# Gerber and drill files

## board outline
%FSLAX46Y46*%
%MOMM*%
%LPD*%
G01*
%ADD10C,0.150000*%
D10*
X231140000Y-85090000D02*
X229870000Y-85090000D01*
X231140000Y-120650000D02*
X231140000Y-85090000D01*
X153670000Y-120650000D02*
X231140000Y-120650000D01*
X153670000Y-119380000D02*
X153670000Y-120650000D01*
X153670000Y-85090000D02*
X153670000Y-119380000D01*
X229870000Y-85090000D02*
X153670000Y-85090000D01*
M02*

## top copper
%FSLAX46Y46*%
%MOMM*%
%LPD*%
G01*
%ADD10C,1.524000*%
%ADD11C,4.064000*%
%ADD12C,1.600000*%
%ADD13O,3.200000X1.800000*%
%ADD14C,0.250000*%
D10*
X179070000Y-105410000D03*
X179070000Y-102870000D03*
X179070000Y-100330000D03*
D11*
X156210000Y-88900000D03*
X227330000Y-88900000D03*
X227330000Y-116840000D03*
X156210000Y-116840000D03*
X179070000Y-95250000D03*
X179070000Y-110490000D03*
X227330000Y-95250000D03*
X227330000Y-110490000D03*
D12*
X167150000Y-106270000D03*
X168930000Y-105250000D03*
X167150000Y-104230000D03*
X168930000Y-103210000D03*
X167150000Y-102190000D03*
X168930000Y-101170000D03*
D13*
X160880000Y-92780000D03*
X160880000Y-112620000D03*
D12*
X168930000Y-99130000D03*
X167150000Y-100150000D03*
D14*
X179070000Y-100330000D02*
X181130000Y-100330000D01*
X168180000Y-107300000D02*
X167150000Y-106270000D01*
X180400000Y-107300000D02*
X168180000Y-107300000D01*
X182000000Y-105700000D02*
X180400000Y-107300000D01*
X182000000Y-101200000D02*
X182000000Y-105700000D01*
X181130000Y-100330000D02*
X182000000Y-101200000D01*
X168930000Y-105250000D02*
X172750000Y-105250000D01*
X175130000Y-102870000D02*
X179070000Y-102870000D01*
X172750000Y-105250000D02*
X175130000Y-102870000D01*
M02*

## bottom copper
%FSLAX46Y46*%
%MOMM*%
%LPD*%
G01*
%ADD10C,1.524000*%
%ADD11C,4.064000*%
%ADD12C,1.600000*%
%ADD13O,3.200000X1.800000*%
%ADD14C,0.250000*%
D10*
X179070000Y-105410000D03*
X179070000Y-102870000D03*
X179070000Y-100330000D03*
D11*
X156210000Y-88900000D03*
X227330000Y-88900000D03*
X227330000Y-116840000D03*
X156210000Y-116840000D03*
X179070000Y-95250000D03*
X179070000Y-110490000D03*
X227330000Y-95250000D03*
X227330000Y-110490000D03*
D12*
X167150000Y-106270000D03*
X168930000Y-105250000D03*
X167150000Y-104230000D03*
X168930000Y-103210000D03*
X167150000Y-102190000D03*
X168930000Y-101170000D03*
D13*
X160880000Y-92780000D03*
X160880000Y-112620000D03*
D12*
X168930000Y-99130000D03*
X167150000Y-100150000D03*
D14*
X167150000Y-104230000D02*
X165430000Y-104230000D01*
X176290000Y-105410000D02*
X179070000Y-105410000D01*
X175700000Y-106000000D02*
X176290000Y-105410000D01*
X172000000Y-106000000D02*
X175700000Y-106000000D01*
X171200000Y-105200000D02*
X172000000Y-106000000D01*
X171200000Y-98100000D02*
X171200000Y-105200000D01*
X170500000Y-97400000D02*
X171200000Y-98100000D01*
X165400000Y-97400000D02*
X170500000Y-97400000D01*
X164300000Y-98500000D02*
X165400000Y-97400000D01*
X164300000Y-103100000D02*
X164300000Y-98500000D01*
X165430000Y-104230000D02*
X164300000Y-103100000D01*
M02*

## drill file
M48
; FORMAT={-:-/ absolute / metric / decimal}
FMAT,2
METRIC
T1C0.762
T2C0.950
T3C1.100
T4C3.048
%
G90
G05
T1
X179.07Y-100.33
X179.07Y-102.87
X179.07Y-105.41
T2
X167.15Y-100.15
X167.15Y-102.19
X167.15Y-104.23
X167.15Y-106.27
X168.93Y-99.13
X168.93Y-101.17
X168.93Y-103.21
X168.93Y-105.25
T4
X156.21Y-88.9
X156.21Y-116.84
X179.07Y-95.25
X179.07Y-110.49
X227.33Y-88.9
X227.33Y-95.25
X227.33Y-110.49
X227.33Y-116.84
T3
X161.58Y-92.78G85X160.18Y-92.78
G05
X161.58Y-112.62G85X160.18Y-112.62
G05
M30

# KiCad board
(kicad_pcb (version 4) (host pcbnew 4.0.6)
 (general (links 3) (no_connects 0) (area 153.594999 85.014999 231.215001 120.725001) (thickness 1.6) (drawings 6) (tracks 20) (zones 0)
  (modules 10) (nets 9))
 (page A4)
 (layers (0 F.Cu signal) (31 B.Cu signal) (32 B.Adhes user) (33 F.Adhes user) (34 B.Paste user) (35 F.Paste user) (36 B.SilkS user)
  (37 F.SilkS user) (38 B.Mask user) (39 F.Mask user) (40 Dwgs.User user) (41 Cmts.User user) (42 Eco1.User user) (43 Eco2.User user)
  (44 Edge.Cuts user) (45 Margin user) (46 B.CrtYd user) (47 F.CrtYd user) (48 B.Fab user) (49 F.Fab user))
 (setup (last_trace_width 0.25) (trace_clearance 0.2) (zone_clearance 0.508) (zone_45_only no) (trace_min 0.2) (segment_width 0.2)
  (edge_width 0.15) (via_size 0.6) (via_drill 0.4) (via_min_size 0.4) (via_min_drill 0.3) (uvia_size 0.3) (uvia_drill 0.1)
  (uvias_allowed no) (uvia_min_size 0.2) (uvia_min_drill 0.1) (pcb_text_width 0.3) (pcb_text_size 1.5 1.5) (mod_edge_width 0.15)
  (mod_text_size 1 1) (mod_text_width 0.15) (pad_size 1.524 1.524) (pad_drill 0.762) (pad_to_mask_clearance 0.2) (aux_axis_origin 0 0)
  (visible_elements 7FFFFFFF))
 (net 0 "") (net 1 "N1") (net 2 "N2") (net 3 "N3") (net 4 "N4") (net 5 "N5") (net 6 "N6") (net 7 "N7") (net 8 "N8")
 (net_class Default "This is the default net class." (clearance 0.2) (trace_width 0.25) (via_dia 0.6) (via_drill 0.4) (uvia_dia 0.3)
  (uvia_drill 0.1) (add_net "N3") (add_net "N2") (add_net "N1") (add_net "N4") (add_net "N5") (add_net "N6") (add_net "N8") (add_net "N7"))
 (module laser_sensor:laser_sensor (layer F.Cu) (at 176.53 102.87)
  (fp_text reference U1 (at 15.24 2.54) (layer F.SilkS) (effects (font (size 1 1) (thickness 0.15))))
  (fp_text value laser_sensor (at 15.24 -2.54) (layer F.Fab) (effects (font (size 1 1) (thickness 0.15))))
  (pad 1 thru_hole circle (at 2.54 2.54) (size 1.524 1.524) (drill 0.762) (layers *.Cu *.Mask) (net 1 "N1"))
  (pad 2 thru_hole circle (at 2.54 0) (size 1.524 1.524) (drill 0.762) (layers *.Cu *.Mask) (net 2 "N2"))
  (pad 3 thru_hole circle (at 2.54 -2.54) (size 1.524 1.524) (drill 0.762) (layers *.Cu *.Mask) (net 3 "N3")))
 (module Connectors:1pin (layer F.Cu) (at 156.21 88.9)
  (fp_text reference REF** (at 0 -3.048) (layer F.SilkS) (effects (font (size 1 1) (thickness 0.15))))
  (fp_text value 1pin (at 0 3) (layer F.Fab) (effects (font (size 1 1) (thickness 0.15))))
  (pad 1 thru_hole circle (at 0 0) (size 4.064 4.064) (drill 3.048) (layers *.Cu *.Mask)))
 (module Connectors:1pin (layer F.Cu) (at 227.33 88.9)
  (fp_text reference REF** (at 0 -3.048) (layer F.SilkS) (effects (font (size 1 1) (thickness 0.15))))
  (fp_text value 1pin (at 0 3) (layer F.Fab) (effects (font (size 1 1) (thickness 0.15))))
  (pad 1 thru_hole circle (at 0 0) (size 4.064 4.064) (drill 3.048) (layers *.Cu *.Mask)))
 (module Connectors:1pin (layer F.Cu) (at 227.33 116.84)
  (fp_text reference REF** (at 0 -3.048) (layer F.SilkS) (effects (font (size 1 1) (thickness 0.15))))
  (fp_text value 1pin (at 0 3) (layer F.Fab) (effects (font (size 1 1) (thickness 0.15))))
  (pad 1 thru_hole circle (at 0 0) (size 4.064 4.064) (drill 3.048) (layers *.Cu *.Mask)))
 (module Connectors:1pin (layer F.Cu) (at 156.21 116.84)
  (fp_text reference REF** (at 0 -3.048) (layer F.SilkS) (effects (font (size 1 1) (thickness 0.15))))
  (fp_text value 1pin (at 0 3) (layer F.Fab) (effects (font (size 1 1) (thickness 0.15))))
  (pad 1 thru_hole circle (at 0 0) (size 4.064 4.064) (drill 3.048) (layers *.Cu *.Mask)))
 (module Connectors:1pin (layer F.Cu) (at 179.07 95.25)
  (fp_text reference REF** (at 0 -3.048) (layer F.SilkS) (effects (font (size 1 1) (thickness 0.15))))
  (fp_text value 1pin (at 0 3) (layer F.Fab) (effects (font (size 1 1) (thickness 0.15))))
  (pad 1 thru_hole circle (at 0 0) (size 4.064 4.064) (drill 3.048) (layers *.Cu *.Mask)))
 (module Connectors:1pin (layer F.Cu) (at 179.07 110.49)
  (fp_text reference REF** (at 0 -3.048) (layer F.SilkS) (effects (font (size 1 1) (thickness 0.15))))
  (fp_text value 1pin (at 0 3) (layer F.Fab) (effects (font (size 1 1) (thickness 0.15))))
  (pad 1 thru_hole circle (at 0 0) (size 4.064 4.064) (drill 3.048) (layers *.Cu *.Mask)))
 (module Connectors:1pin (layer F.Cu) (at 227.33 95.25)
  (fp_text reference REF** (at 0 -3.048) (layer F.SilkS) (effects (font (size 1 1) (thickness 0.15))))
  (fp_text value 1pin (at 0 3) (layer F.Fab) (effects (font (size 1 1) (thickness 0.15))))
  (pad 1 thru_hole circle (at 0 0) (size 4.064 4.064) (drill 3.048) (layers *.Cu *.Mask)))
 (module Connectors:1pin (layer F.Cu) (at 227.33 110.49)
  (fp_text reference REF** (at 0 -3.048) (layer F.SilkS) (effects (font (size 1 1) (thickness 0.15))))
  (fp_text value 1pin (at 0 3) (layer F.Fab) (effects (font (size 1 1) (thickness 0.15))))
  (pad 1 thru_hole circle (at 0 0) (size 4.064 4.064) (drill 3.048) (layers *.Cu *.Mask)))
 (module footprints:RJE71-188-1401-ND (layer F.Cu) (at 172.6 94.6 270)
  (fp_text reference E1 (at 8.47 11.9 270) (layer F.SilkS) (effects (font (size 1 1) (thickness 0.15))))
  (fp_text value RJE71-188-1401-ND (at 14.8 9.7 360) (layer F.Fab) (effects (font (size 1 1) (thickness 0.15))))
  (pad 1 thru_hole circle (at 11.67 5.45 270) (size 1.6 1.6) (drill 0.95) (layers *.Cu *.Mask) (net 3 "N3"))
  (pad 2 thru_hole circle (at 10.65 3.67 270) (size 1.6 1.6) (drill 0.95) (layers *.Cu *.Mask) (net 2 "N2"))
  (pad 3 thru_hole circle (at 9.63 5.45 270) (size 1.6 1.6) (drill 0.95) (layers *.Cu *.Mask) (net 1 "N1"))
  (pad 4 thru_hole circle (at 8.61 3.67 270) (size 1.6 1.6) (drill 0.95) (layers *.Cu *.Mask) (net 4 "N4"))
  (pad 5 thru_hole circle (at 7.59 5.45 270) (size 1.6 1.6) (drill 0.95) (layers *.Cu *.Mask) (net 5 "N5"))
  (pad 6 thru_hole circle (at 6.57 3.67 270) (size 1.6 1.6) (drill 0.95) (layers *.Cu *.Mask) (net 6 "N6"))
  (pad "" thru_hole oval (at -1.82 11.72 270) (size 1.8 3.2) (drill oval 1.1 2.5) (layers *.Cu *.Mask))
  (pad "" thru_hole oval (at 18.02 11.72 270) (size 1.8 3.2) (drill oval 1.1 2.5) (layers *.Cu *.Mask))
  (pad 8 thru_hole circle (at 4.53 3.67 270) (size 1.6 1.6) (drill 0.95) (layers *.Cu *.Mask) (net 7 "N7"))
  (pad 7 thru_hole circle (at 5.55 5.45 270) (size 1.6 1.6) (drill 0.95) (layers *.Cu *.Mask) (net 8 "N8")))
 (gr_line (start 231.14 85.09) (end 229.87 85.09) (angle 90) (layer Edge.Cuts) (width 0.15))
 (gr_line (start 231.14 120.65) (end 231.14 85.09) (angle 90) (layer Edge.Cuts) (width 0.15))
 (gr_line (start 153.67 120.65) (end 231.14 120.65) (angle 90) (layer Edge.Cuts) (width 0.15))
 (gr_line (start 153.67 119.38) (end 153.67 120.65) (angle 90) (layer Edge.Cuts) (width 0.15))
 (gr_line (start 153.67 85.09) (end 153.67 119.38) (angle 90) (layer Edge.Cuts) (width 0.15))
 (gr_line (start 229.87 85.09) (end 153.67 85.09) (angle 90) (layer Edge.Cuts) (width 0.15))
 (segment (start 179.07 100.33) (end 181.13 100.33) (width 0.25) (layer F.Cu) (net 3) (status 400000))
 (segment (start 168.18 107.3) (end 167.15 106.27) (width 0.25) (layer F.Cu) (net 3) (status 800000))
 (segment (start 180.4 107.3) (end 168.18 107.3) (width 0.25) (layer F.Cu) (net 3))
 (segment (start 182 105.7) (end 180.4 107.3) (width 0.25) (layer F.Cu) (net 3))
 (segment (start 182 101.2) (end 182 105.7) (width 0.25) (layer F.Cu) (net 3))
 (segment (start 181.13 100.33) (end 182 101.2) (width 0.25) (layer F.Cu) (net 3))
 (segment (start 168.93 105.25) (end 172.75 105.25) (width 0.25) (layer F.Cu) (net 2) (status 400000))
 (segment (start 175.13 102.87) (end 179.07 102.87) (width 0.25) (layer F.Cu) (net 2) (status 800000))
 (segment (start 172.75 105.25) (end 175.13 102.87) (width 0.25) (layer F.Cu) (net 2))
 (segment (start 167.15 104.23) (end 165.43 104.23) (width 0.25) (layer B.Cu) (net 1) (status 400000))
 (segment (start 176.29 105.41) (end 179.07 105.41) (width 0.25) (layer B.Cu) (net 1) (status 800000))
 (segment (start 175.7 106) (end 176.29 105.41) (width 0.25) (layer B.Cu) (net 1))
 (segment (start 172 106) (end 175.7 106) (width 0.25) (layer B.Cu) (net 1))
 (segment (start 171.2 105.2) (end 172 106) (width 0.25) (layer B.Cu) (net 1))
 (segment (start 171.2 98.1) (end 171.2 105.2) (width 0.25) (layer B.Cu) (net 1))
 (segment (start 170.5 97.4) (end 171.2 98.1) (width 0.25) (layer B.Cu) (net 1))
 (segment (start 165.4 97.4) (end 170.5 97.4) (width 0.25) (layer B.Cu) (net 1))
 (segment (start 164.3 98.5) (end 165.4 97.4) (width 0.25) (layer B.Cu) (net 1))
 (segment (start 164.3 103.1) (end 164.3 98.5) (width 0.25) (layer B.Cu) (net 1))
 (segment (start 165.43 104.23) (end 164.3 103.1) (width 0.25) (layer B.Cu) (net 1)))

